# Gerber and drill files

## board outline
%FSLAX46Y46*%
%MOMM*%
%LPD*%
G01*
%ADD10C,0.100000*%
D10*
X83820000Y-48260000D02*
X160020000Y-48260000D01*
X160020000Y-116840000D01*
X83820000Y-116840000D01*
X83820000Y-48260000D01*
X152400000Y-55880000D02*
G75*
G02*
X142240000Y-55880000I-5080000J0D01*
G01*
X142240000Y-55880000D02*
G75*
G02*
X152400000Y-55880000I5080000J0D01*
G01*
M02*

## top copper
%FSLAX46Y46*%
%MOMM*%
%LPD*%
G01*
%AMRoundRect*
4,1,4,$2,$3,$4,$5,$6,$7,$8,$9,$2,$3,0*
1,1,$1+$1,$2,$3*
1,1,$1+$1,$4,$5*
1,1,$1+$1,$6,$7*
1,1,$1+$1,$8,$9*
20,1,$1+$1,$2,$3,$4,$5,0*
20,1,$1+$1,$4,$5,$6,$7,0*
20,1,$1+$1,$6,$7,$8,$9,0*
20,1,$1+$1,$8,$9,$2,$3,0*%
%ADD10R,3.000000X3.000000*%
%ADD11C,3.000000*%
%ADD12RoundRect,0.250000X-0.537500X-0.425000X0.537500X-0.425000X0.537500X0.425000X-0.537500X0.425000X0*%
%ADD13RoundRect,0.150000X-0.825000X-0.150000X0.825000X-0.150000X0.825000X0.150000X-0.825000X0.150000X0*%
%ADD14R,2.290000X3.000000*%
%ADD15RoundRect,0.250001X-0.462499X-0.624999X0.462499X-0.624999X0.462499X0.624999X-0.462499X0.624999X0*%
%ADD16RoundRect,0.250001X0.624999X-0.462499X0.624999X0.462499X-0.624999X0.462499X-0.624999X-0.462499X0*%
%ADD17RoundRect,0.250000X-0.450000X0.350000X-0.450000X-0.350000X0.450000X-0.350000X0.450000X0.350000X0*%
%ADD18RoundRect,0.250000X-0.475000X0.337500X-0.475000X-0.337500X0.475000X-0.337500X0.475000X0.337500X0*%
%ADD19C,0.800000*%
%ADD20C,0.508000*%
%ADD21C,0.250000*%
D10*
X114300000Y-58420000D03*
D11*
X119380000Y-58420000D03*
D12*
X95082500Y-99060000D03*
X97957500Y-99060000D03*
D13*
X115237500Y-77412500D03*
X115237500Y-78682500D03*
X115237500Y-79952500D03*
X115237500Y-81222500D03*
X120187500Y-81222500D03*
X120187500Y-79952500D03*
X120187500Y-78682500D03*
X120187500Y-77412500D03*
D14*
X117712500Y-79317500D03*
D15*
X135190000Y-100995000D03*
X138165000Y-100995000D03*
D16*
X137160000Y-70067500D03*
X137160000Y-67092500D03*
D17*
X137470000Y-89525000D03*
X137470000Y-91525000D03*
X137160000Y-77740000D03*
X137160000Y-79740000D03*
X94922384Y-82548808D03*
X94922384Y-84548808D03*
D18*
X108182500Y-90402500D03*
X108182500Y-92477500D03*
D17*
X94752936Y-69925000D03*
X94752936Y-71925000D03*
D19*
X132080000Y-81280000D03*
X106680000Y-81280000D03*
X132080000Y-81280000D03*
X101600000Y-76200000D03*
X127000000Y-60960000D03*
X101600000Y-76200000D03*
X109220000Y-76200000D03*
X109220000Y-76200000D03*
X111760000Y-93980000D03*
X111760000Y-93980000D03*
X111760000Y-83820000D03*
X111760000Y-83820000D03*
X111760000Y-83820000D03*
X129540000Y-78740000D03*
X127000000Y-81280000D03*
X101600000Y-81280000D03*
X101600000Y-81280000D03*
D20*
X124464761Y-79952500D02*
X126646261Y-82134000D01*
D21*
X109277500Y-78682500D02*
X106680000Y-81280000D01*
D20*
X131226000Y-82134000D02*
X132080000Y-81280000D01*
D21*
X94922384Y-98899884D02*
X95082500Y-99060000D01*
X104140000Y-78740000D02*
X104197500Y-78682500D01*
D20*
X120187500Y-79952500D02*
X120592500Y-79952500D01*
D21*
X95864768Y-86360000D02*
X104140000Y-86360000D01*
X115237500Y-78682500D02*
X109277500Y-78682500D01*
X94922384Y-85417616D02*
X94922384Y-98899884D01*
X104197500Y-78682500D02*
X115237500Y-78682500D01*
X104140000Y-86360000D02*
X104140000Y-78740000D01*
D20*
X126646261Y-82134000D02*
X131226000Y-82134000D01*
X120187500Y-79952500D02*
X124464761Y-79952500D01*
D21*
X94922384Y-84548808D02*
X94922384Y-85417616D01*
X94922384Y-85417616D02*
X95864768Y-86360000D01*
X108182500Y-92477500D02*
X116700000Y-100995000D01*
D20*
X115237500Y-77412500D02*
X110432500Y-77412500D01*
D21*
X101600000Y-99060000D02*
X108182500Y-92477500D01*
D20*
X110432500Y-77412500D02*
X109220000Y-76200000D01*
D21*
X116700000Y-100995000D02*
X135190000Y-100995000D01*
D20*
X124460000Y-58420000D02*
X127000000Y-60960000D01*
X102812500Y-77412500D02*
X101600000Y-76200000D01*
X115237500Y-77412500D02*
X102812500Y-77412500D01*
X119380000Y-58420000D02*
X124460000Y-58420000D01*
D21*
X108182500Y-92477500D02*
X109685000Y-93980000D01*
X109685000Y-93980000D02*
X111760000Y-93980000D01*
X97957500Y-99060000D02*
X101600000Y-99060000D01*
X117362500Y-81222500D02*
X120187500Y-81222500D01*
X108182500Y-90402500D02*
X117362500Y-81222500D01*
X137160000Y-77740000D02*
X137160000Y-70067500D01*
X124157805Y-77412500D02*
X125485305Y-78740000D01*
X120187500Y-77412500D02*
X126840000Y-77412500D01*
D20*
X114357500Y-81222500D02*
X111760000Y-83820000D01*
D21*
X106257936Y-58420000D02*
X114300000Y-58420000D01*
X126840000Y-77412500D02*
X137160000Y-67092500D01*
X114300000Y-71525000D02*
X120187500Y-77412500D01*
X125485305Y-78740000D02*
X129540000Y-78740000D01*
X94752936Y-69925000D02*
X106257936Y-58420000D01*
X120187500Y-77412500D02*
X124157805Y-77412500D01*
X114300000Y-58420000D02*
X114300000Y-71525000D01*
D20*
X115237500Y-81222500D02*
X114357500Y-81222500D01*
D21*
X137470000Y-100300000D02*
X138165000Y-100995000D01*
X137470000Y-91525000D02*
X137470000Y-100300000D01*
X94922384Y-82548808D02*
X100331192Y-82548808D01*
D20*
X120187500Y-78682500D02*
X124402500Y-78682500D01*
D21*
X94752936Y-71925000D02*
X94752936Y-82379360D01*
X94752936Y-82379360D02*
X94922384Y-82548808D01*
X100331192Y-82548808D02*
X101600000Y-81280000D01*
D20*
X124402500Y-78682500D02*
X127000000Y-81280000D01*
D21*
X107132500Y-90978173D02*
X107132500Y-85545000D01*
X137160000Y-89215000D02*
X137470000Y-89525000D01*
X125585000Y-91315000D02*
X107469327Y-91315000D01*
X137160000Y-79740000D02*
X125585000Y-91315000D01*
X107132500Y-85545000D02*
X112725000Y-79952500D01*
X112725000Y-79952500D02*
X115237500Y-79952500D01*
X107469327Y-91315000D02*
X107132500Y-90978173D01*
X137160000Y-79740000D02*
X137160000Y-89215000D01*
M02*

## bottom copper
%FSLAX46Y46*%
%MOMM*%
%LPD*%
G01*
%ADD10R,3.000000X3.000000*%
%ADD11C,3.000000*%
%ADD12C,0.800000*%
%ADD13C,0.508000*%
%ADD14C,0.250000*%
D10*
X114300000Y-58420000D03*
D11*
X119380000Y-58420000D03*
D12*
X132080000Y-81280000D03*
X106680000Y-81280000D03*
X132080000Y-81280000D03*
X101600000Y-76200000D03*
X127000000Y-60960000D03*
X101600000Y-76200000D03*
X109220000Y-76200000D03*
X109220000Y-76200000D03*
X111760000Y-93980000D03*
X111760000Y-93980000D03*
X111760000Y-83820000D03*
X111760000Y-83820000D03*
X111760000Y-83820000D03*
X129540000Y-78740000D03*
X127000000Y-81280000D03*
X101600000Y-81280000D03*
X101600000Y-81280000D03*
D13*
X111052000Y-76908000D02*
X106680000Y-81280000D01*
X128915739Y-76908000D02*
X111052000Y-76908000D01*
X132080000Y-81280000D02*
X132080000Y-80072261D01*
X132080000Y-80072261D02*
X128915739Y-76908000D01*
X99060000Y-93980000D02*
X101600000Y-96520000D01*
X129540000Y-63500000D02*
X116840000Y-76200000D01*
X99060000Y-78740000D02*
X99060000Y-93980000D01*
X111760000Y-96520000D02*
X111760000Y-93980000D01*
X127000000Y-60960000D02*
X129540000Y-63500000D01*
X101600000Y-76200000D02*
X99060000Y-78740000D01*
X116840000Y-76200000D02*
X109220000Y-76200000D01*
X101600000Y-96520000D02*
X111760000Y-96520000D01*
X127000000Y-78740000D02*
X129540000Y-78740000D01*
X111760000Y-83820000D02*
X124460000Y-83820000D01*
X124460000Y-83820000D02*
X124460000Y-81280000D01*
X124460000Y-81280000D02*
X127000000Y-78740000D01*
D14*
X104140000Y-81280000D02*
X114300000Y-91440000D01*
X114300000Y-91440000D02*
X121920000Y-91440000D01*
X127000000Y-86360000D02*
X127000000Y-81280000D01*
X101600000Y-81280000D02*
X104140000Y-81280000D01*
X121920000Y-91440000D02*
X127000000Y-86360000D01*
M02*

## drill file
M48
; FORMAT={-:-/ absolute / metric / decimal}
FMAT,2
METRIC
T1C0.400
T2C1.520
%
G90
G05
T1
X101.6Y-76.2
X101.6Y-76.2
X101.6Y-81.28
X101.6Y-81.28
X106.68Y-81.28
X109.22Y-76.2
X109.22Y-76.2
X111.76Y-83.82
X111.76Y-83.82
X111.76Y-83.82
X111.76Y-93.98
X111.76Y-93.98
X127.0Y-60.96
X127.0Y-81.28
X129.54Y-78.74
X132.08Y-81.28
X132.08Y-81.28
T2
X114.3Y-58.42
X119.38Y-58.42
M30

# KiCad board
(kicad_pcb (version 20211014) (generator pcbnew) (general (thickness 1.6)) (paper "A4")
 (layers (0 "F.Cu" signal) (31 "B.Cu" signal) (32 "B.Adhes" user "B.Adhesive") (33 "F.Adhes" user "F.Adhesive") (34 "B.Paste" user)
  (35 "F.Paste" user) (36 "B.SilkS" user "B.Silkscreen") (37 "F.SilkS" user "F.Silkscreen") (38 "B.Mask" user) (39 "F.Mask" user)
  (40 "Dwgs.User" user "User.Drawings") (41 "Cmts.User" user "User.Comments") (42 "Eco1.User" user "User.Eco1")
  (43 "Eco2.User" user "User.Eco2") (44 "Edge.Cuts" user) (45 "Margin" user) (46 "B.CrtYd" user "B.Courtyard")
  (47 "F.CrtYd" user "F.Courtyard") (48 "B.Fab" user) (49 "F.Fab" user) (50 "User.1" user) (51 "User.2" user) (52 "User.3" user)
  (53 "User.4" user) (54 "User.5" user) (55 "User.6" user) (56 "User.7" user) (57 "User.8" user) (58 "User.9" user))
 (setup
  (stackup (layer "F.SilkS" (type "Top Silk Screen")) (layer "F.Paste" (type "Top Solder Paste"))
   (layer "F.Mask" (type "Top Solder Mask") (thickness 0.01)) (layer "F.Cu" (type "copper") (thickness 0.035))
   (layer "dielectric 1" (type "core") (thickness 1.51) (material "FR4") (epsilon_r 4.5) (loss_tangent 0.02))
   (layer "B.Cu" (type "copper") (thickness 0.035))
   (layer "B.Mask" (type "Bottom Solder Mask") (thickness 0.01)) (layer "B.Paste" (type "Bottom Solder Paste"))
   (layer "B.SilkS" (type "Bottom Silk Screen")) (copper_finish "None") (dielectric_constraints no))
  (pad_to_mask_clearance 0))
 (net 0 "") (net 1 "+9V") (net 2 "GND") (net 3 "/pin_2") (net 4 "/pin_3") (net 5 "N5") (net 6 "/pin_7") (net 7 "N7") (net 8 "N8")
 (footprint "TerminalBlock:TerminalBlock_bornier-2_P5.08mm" (layer "F.Cu") (at 114.3 58.42)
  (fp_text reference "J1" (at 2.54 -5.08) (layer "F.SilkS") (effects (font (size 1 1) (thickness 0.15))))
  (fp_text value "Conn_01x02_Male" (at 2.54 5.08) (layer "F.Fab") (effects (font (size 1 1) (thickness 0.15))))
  (pad "1" thru_hole rect (at 0 0) (size 3 3) (drill 1.52) (layers *.Cu *.Mask) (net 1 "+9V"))
  (pad "2" thru_hole circle (at 5.08 0) (size 3 3) (drill 1.52) (layers *.Cu *.Mask) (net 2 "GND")))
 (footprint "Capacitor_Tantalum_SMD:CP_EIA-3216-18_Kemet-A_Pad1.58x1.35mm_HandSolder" (layer "F.Cu") (at 96.52 99.06)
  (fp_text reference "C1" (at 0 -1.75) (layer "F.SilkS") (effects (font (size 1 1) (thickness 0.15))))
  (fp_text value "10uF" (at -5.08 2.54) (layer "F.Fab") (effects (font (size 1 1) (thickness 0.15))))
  (pad "1" smd roundrect (at -1.4375 0) (size 1.575 1.35) (layers "F.Cu" "F.Paste" "F.Mask") (roundrect_rratio 0.185185) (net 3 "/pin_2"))
  (pad "2" smd roundrect (at 1.4375 0) (size 1.575 1.35) (layers "F.Cu" "F.Paste" "F.Mask") (roundrect_rratio 0.185185) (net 2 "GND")))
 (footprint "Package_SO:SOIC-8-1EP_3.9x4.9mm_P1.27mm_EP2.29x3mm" (layer "F.Cu") (at 117.7125 79.3175)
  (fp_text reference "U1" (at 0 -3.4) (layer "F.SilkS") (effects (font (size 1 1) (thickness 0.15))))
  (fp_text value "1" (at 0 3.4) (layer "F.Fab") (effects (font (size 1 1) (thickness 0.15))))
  (pad "" smd roundrect (at 0.57 0.75) (size 0.92 1.21) (layers "F.Paste") (roundrect_rratio 0.25))
  (pad "" smd roundrect (at -0.57 -0.75) (size 0.92 1.21) (layers "F.Paste") (roundrect_rratio 0.25))
  (pad "" smd roundrect (at -0.57 0.75) (size 0.92 1.21) (layers "F.Paste") (roundrect_rratio 0.25))
  (pad "" smd roundrect (at 0.57 -0.75) (size 0.92 1.21) (layers "F.Paste") (roundrect_rratio 0.25))
  (pad "1" smd roundrect (at -2.475 -1.905) (size 1.95 0.6) (layers "F.Cu" "F.Paste" "F.Mask") (roundrect_rratio 0.25) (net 2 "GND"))
  (pad "2" smd roundrect (at -2.475 -0.635) (size 1.95 0.6) (layers "F.Cu" "F.Paste" "F.Mask") (roundrect_rratio 0.25) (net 3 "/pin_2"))
  (pad "3" smd roundrect (at -2.475 0.635) (size 1.95 0.6) (layers "F.Cu" "F.Paste" "F.Mask") (roundrect_rratio 0.25) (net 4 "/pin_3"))
  (pad "4" smd roundrect (at -2.475 1.905) (size 1.95 0.6) (layers "F.Cu" "F.Paste" "F.Mask") (roundrect_rratio 0.25) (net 1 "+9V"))
  (pad "5" smd roundrect (at 2.475 1.905) (size 1.95 0.6) (layers "F.Cu" "F.Paste" "F.Mask") (roundrect_rratio 0.25) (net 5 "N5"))
  (pad "6" smd roundrect (at 2.475 0.635) (size 1.95 0.6) (layers "F.Cu" "F.Paste" "F.Mask") (roundrect_rratio 0.25) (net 3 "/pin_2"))
  (pad "7" smd roundrect (at 2.475 -0.635) (size 1.95 0.6) (layers "F.Cu" "F.Paste" "F.Mask") (roundrect_rratio 0.25) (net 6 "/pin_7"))
  (pad "8" smd roundrect (at 2.475 -1.905) (size 1.95 0.6) (layers "F.Cu" "F.Paste" "F.Mask") (roundrect_rratio 0.25) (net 1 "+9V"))
  (pad "9" smd rect (at 0 0) (size 2.29 3) (layers "F.Cu" "F.Mask")))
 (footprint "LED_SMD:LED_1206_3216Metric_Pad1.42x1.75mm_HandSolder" (layer "F.Cu") (at 136.6775 100.995)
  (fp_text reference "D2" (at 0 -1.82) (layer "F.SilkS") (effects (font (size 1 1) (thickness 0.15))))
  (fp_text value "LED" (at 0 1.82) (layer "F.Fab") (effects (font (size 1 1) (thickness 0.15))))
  (pad "1" smd roundrect (at -1.4875 0) (size 1.425 1.75) (layers "F.Cu" "F.Paste" "F.Mask") (roundrect_rratio 0.175439) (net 2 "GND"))
  (pad "2" smd roundrect (at 1.4875 0) (size 1.425 1.75) (layers "F.Cu" "F.Paste" "F.Mask") (roundrect_rratio 0.175439) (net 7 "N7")))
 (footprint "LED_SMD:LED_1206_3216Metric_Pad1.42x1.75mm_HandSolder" (layer "F.Cu") (at 137.16 68.58 90)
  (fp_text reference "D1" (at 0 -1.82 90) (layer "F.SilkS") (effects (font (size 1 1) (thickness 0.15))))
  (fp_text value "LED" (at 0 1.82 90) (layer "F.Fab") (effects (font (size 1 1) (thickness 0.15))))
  (pad "1" smd roundrect (at -1.4875 0 90) (size 1.425 1.75) (layers "F.Cu" "F.Paste" "F.Mask") (roundrect_rratio 0.175439) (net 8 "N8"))
  (pad "2" smd roundrect (at 1.4875 0 90) (size 1.425 1.75) (layers "F.Cu" "F.Paste" "F.Mask") (roundrect_rratio 0.175439) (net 1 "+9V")))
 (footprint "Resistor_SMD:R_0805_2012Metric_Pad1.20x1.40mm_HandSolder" (layer "F.Cu") (at 137.47 90.525 -90)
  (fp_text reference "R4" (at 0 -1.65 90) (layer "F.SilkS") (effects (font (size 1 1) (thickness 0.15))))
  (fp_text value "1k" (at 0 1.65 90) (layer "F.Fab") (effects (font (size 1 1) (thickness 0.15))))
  (pad "1" smd roundrect (at -1 0 270) (size 1.2 1.4) (layers "F.Cu" "F.Paste" "F.Mask") (roundrect_rratio 0.208333) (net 4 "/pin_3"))
  (pad "2" smd roundrect (at 1 0 270) (size 1.2 1.4) (layers "F.Cu" "F.Paste" "F.Mask") (roundrect_rratio 0.208333) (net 7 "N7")))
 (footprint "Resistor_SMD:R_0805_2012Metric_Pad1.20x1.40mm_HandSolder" (layer "F.Cu") (at 137.16 78.74 -90)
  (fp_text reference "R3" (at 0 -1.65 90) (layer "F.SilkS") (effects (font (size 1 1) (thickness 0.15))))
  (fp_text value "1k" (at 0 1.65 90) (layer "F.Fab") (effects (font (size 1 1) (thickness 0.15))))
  (pad "1" smd roundrect (at -1 0 270) (size 1.2 1.4) (layers "F.Cu" "F.Paste" "F.Mask") (roundrect_rratio 0.208333) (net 8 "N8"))
  (pad "2" smd roundrect (at 1 0 270) (size 1.2 1.4) (layers "F.Cu" "F.Paste" "F.Mask") (roundrect_rratio 0.208333) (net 4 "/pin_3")))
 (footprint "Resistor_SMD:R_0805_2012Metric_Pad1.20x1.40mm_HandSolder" (layer "F.Cu") (at 94.922384 83.548808 -90)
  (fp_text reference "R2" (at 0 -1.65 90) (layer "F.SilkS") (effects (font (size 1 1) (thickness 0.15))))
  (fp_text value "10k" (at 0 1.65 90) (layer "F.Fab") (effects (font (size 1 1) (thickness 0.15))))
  (pad "1" smd roundrect (at -1 0 270) (size 1.2 1.4) (layers "F.Cu" "F.Paste" "F.Mask") (roundrect_rratio 0.208333) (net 6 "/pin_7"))
  (pad "2" smd roundrect (at 1 0 270) (size 1.2 1.4) (layers "F.Cu" "F.Paste" "F.Mask") (roundrect_rratio 0.208333) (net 3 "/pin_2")))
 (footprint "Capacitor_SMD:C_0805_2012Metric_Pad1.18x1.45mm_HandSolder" (layer "F.Cu") (at 108.1825 91.44 -90)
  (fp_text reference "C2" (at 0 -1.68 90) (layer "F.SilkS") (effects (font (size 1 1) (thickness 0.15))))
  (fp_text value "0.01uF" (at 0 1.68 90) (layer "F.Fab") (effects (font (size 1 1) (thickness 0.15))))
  (pad "1" smd roundrect (at -1.0375 0 270) (size 1.175 1.45) (layers "F.Cu" "F.Paste" "F.Mask") (roundrect_rratio 0.212766) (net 5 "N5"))
  (pad "2" smd roundrect (at 1.0375 0 270) (size 1.175 1.45) (layers "F.Cu" "F.Paste" "F.Mask") (roundrect_rratio 0.212766) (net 2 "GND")))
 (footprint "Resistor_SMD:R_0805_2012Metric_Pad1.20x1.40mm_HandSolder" (layer "F.Cu") (at 94.752936 70.925 -90)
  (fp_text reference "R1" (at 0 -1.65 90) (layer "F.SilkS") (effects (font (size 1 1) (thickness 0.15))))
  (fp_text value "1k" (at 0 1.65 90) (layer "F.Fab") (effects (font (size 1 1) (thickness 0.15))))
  (pad "1" smd roundrect (at -1 0 270) (size 1.2 1.4) (layers "F.Cu" "F.Paste" "F.Mask") (roundrect_rratio 0.208333) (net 1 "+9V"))
  (pad "2" smd roundrect (at 1 0 270) (size 1.2 1.4) (layers "F.Cu" "F.Paste" "F.Mask") (roundrect_rratio 0.208333) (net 6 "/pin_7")))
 (gr_rect (start 83.82 48.26) (end 160.02 116.84) (layer "Edge.Cuts") (width 0.1) (fill none))
 (gr_circle (center 147.32 55.88) (end 152.4 55.88) (layer "Edge.Cuts") (width 0.1) (fill none))
 (segment (start 124.464761 79.9525) (end 126.646261 82.134) (width 0.508) (layer "F.Cu") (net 3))
 (segment (start 109.2775 78.6825) (end 106.68 81.28) (width 0.25) (layer "F.Cu") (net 3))
 (segment (start 131.226 82.134) (end 132.08 81.28) (width 0.508) (layer "F.Cu") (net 3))
 (segment (start 94.922384 98.899884) (end 95.0825 99.06) (width 0.25) (layer "F.Cu") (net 3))
 (segment (start 104.14 78.74) (end 104.1975 78.6825) (width 0.25) (layer "F.Cu") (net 3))
 (segment (start 120.1875 79.9525) (end 120.5925 79.9525) (width 0.508) (layer "F.Cu") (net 3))
 (segment (start 95.864768 86.36) (end 104.14 86.36) (width 0.25) (layer "F.Cu") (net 3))
 (segment (start 115.2375 78.6825) (end 109.2775 78.6825) (width 0.25) (layer "F.Cu") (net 3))
 (segment (start 94.922384 85.417616) (end 94.922384 98.899884) (width 0.25) (layer "F.Cu") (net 3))
 (segment (start 104.1975 78.6825) (end 115.2375 78.6825) (width 0.25) (layer "F.Cu") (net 3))
 (segment (start 104.14 86.36) (end 104.14 78.74) (width 0.25) (layer "F.Cu") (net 3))
 (segment (start 126.646261 82.134) (end 131.226 82.134) (width 0.508) (layer "F.Cu") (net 3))
 (segment (start 120.1875 79.9525) (end 124.464761 79.9525) (width 0.508) (layer "F.Cu") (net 3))
 (segment (start 94.922384 84.548808) (end 94.922384 85.417616) (width 0.25) (layer "F.Cu") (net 3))
 (segment (start 94.922384 85.417616) (end 95.864768 86.36) (width 0.25) (layer "F.Cu") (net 3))
 (via (at 132.08 81.28) (size 0.8) (drill 0.4) (layers "F.Cu" "B.Cu") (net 3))
 (via (at 106.68 81.28) (size 0.8) (drill 0.4) (layers "F.Cu" "B.Cu") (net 3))
 (via (at 132.08 81.28) (size 0.8) (drill 0.4) (layers "F.Cu" "B.Cu") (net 3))
 (segment (start 111.052 76.908) (end 106.68 81.28) (width 0.508) (layer "B.Cu") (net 3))
 (segment (start 128.915739 76.908) (end 111.052 76.908) (width 0.508) (layer "B.Cu") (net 3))
 (segment (start 132.08 81.28) (end 132.08 80.072261) (width 0.508) (layer "B.Cu") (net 3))
 (segment (start 132.08 80.072261) (end 128.915739 76.908) (width 0.508) (layer "B.Cu") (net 3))
 (segment (start 108.1825 92.4775) (end 116.7 100.995) (width 0.25) (layer "F.Cu") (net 2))
 (segment (start 115.2375 77.4125) (end 110.4325 77.4125) (width 0.508) (layer "F.Cu") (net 2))
 (segment (start 101.6 99.06) (end 108.1825 92.4775) (width 0.25) (layer "F.Cu") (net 2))
 (segment (start 110.4325 77.4125) (end 109.22 76.2) (width 0.508) (layer "F.Cu") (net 2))
 (segment (start 116.7 100.995) (end 135.19 100.995) (width 0.25) (layer "F.Cu") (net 2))
 (segment (start 124.46 58.42) (end 127 60.96) (width 0.508) (layer "F.Cu") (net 2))
 (segment (start 102.8125 77.4125) (end 101.6 76.2) (width 0.508) (layer "F.Cu") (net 2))
 (segment (start 115.2375 77.4125) (end 102.8125 77.4125) (width 0.508) (layer "F.Cu") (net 2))
 (segment (start 119.38 58.42) (end 124.46 58.42) (width 0.508) (layer "F.Cu") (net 2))
 (segment (start 108.1825 92.4775) (end 109.685 93.98) (width 0.25) (layer "F.Cu") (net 2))
 (segment (start 109.685 93.98) (end 111.76 93.98) (width 0.25) (layer "F.Cu") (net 2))
 (segment (start 97.9575 99.06) (end 101.6 99.06) (width 0.25) (layer "F.Cu") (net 2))
 (via (at 101.6 76.2) (size 0.8) (drill 0.4) (layers "F.Cu" "B.Cu") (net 2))
 (via (at 127 60.96) (size 0.8) (drill 0.4) (layers "F.Cu" "B.Cu") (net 2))
 (via (at 101.6 76.2) (size 0.8) (drill 0.4) (layers "F.Cu" "B.Cu") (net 2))
 (via (at 109.22 76.2) (size 0.8) (drill 0.4) (layers "F.Cu" "B.Cu") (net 2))
 (via (at 109.22 76.2) (size 0.8) (drill 0.4) (layers "F.Cu" "B.Cu") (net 2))
 (via (at 111.76 93.98) (size 0.8) (drill 0.4) (layers "F.Cu" "B.Cu") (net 2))
 (via (at 111.76 93.98) (size 0.8) (drill 0.4) (layers "F.Cu" "B.Cu") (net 2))
 (segment (start 99.06 93.98) (end 101.6 96.52) (width 0.508) (layer "B.Cu") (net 2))
 (segment (start 129.54 63.5) (end 116.84 76.2) (width 0.508) (layer "B.Cu") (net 2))
 (segment (start 99.06 78.74) (end 99.06 93.98) (width 0.508) (layer "B.Cu") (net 2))
 (segment (start 111.76 96.52) (end 111.76 93.98) (width 0.508) (layer "B.Cu") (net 2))
 (segment (start 127 60.96) (end 129.54 63.5) (width 0.508) (layer "B.Cu") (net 2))
 (segment (start 101.6 76.2) (end 99.06 78.74) (width 0.508) (layer "B.Cu") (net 2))
 (segment (start 116.84 76.2) (end 109.22 76.2) (width 0.508) (layer "B.Cu") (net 2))
 (segment (start 101.6 96.52) (end 111.76 96.52) (width 0.508) (layer "B.Cu") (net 2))
 (segment (start 117.3625 81.2225) (end 120.1875 81.2225) (width 0.25) (layer "F.Cu") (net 5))
 (segment (start 108.1825 90.4025) (end 117.3625 81.2225) (width 0.25) (layer "F.Cu") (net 5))
 (segment (start 137.16 77.74) (end 137.16 70.0675) (width 0.25) (layer "F.Cu") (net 8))
 (segment (start 124.157805 77.4125) (end 125.485305 78.74) (width 0.25) (layer "F.Cu") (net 1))
 (segment (start 120.1875 77.4125) (end 126.84 77.4125) (width 0.25) (layer "F.Cu") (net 1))
 (segment (start 114.3575 81.2225) (end 111.76 83.82) (width 0.508) (layer "F.Cu") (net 1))
 (segment (start 106.257936 58.42) (end 114.3 58.42) (width 0.25) (layer "F.Cu") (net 1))
 (segment (start 126.84 77.4125) (end 137.16 67.0925) (width 0.25) (layer "F.Cu") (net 1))
 (segment (start 114.3 71.525) (end 120.1875 77.4125) (width 0.25) (layer "F.Cu") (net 1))
 (segment (start 125.485305 78.74) (end 129.54 78.74) (width 0.25) (layer "F.Cu") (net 1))
 (segment (start 94.752936 69.925) (end 106.257936 58.42) (width 0.25) (layer "F.Cu") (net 1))
 (segment (start 120.1875 77.4125) (end 124.157805 77.4125) (width 0.25) (layer "F.Cu") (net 1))
 (segment (start 114.3 58.42) (end 114.3 71.525) (width 0.25) (layer "F.Cu") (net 1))
 (segment (start 115.2375 81.2225) (end 114.3575 81.2225) (width 0.508) (layer "F.Cu") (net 1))
 (via (at 111.76 83.82) (size 0.8) (drill 0.4) (layers "F.Cu" "B.Cu") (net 1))
 (via (at 111.76 83.82) (size 0.8) (drill 0.4) (layers "F.Cu" "B.Cu") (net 1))
 (via (at 111.76 83.82) (size 0.8) (drill 0.4) (layers "F.Cu" "B.Cu") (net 1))
 (via (at 129.54 78.74) (size 0.8) (drill 0.4) (layers "F.Cu" "B.Cu") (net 1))
 (segment (start 127 78.74) (end 129.54 78.74) (width 0.508) (layer "B.Cu") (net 1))
 (segment (start 111.76 83.82) (end 124.46 83.82) (width 0.508) (layer "B.Cu") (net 1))
 (segment (start 124.46 83.82) (end 124.46 81.28) (width 0.508) (layer "B.Cu") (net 1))
 (segment (start 124.46 81.28) (end 127 78.74) (width 0.508) (layer "B.Cu") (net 1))
 (segment (start 137.47 100.3) (end 138.165 100.995) (width 0.25) (layer "F.Cu") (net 7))
 (segment (start 137.47 91.525) (end 137.47 100.3) (width 0.25) (layer "F.Cu") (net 7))
 (segment (start 94.922384 82.548808) (end 100.331192 82.548808) (width 0.25) (layer "F.Cu") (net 6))
 (segment (start 120.1875 78.6825) (end 124.4025 78.6825) (width 0.508) (layer "F.Cu") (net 6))
 (segment (start 94.752936 71.925) (end 94.752936 82.37936) (width 0.25) (layer "F.Cu") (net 6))
 (segment (start 94.752936 82.37936) (end 94.922384 82.548808) (width 0.25) (layer "F.Cu") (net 6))
 (segment (start 100.331192 82.548808) (end 101.6 81.28) (width 0.25) (layer "F.Cu") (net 6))
 (segment (start 124.4025 78.6825) (end 127 81.28) (width 0.508) (layer "F.Cu") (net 6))
 (via (at 127 81.28) (size 0.8) (drill 0.4) (layers "F.Cu" "B.Cu") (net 6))
 (via (at 101.6 81.28) (size 0.8) (drill 0.4) (layers "F.Cu" "B.Cu") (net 6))
 (via (at 101.6 81.28) (size 0.8) (drill 0.4) (layers "F.Cu" "B.Cu") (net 6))
 (segment (start 104.14 81.28) (end 114.3 91.44) (width 0.25) (layer "B.Cu") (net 6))
 (segment (start 114.3 91.44) (end 121.92 91.44) (width 0.25) (layer "B.Cu") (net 6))
 (segment (start 127 86.36) (end 127 81.28) (width 0.25) (layer "B.Cu") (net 6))
 (segment (start 101.6 81.28) (end 104.14 81.28) (width 0.25) (layer "B.Cu") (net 6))
 (segment (start 121.92 91.44) (end 127 86.36) (width 0.25) (layer "B.Cu") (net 6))
 (segment (start 107.1325 90.978173) (end 107.1325 85.545) (width 0.25) (layer "F.Cu") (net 4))
 (segment (start 137.16 89.215) (end 137.47 89.525) (width 0.25) (layer "F.Cu") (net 4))
 (segment (start 125.585 91.315) (end 107.469327 91.315) (width 0.25) (layer "F.Cu") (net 4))
 (segment (start 137.16 79.74) (end 125.585 91.315) (width 0.25) (layer "F.Cu") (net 4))
 (segment (start 107.1325 85.545) (end 112.725 79.9525) (width 0.25) (layer "F.Cu") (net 4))
 (segment (start 112.725 79.9525) (end 115.2375 79.9525) (width 0.25) (layer "F.Cu") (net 4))
 (segment (start 107.469327 91.315) (end 107.1325 90.978173) (width 0.25) (layer "F.Cu") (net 4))
 (segment (start 137.16 79.74) (end 137.16 89.215) (width 0.25) (layer "F.Cu") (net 4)))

